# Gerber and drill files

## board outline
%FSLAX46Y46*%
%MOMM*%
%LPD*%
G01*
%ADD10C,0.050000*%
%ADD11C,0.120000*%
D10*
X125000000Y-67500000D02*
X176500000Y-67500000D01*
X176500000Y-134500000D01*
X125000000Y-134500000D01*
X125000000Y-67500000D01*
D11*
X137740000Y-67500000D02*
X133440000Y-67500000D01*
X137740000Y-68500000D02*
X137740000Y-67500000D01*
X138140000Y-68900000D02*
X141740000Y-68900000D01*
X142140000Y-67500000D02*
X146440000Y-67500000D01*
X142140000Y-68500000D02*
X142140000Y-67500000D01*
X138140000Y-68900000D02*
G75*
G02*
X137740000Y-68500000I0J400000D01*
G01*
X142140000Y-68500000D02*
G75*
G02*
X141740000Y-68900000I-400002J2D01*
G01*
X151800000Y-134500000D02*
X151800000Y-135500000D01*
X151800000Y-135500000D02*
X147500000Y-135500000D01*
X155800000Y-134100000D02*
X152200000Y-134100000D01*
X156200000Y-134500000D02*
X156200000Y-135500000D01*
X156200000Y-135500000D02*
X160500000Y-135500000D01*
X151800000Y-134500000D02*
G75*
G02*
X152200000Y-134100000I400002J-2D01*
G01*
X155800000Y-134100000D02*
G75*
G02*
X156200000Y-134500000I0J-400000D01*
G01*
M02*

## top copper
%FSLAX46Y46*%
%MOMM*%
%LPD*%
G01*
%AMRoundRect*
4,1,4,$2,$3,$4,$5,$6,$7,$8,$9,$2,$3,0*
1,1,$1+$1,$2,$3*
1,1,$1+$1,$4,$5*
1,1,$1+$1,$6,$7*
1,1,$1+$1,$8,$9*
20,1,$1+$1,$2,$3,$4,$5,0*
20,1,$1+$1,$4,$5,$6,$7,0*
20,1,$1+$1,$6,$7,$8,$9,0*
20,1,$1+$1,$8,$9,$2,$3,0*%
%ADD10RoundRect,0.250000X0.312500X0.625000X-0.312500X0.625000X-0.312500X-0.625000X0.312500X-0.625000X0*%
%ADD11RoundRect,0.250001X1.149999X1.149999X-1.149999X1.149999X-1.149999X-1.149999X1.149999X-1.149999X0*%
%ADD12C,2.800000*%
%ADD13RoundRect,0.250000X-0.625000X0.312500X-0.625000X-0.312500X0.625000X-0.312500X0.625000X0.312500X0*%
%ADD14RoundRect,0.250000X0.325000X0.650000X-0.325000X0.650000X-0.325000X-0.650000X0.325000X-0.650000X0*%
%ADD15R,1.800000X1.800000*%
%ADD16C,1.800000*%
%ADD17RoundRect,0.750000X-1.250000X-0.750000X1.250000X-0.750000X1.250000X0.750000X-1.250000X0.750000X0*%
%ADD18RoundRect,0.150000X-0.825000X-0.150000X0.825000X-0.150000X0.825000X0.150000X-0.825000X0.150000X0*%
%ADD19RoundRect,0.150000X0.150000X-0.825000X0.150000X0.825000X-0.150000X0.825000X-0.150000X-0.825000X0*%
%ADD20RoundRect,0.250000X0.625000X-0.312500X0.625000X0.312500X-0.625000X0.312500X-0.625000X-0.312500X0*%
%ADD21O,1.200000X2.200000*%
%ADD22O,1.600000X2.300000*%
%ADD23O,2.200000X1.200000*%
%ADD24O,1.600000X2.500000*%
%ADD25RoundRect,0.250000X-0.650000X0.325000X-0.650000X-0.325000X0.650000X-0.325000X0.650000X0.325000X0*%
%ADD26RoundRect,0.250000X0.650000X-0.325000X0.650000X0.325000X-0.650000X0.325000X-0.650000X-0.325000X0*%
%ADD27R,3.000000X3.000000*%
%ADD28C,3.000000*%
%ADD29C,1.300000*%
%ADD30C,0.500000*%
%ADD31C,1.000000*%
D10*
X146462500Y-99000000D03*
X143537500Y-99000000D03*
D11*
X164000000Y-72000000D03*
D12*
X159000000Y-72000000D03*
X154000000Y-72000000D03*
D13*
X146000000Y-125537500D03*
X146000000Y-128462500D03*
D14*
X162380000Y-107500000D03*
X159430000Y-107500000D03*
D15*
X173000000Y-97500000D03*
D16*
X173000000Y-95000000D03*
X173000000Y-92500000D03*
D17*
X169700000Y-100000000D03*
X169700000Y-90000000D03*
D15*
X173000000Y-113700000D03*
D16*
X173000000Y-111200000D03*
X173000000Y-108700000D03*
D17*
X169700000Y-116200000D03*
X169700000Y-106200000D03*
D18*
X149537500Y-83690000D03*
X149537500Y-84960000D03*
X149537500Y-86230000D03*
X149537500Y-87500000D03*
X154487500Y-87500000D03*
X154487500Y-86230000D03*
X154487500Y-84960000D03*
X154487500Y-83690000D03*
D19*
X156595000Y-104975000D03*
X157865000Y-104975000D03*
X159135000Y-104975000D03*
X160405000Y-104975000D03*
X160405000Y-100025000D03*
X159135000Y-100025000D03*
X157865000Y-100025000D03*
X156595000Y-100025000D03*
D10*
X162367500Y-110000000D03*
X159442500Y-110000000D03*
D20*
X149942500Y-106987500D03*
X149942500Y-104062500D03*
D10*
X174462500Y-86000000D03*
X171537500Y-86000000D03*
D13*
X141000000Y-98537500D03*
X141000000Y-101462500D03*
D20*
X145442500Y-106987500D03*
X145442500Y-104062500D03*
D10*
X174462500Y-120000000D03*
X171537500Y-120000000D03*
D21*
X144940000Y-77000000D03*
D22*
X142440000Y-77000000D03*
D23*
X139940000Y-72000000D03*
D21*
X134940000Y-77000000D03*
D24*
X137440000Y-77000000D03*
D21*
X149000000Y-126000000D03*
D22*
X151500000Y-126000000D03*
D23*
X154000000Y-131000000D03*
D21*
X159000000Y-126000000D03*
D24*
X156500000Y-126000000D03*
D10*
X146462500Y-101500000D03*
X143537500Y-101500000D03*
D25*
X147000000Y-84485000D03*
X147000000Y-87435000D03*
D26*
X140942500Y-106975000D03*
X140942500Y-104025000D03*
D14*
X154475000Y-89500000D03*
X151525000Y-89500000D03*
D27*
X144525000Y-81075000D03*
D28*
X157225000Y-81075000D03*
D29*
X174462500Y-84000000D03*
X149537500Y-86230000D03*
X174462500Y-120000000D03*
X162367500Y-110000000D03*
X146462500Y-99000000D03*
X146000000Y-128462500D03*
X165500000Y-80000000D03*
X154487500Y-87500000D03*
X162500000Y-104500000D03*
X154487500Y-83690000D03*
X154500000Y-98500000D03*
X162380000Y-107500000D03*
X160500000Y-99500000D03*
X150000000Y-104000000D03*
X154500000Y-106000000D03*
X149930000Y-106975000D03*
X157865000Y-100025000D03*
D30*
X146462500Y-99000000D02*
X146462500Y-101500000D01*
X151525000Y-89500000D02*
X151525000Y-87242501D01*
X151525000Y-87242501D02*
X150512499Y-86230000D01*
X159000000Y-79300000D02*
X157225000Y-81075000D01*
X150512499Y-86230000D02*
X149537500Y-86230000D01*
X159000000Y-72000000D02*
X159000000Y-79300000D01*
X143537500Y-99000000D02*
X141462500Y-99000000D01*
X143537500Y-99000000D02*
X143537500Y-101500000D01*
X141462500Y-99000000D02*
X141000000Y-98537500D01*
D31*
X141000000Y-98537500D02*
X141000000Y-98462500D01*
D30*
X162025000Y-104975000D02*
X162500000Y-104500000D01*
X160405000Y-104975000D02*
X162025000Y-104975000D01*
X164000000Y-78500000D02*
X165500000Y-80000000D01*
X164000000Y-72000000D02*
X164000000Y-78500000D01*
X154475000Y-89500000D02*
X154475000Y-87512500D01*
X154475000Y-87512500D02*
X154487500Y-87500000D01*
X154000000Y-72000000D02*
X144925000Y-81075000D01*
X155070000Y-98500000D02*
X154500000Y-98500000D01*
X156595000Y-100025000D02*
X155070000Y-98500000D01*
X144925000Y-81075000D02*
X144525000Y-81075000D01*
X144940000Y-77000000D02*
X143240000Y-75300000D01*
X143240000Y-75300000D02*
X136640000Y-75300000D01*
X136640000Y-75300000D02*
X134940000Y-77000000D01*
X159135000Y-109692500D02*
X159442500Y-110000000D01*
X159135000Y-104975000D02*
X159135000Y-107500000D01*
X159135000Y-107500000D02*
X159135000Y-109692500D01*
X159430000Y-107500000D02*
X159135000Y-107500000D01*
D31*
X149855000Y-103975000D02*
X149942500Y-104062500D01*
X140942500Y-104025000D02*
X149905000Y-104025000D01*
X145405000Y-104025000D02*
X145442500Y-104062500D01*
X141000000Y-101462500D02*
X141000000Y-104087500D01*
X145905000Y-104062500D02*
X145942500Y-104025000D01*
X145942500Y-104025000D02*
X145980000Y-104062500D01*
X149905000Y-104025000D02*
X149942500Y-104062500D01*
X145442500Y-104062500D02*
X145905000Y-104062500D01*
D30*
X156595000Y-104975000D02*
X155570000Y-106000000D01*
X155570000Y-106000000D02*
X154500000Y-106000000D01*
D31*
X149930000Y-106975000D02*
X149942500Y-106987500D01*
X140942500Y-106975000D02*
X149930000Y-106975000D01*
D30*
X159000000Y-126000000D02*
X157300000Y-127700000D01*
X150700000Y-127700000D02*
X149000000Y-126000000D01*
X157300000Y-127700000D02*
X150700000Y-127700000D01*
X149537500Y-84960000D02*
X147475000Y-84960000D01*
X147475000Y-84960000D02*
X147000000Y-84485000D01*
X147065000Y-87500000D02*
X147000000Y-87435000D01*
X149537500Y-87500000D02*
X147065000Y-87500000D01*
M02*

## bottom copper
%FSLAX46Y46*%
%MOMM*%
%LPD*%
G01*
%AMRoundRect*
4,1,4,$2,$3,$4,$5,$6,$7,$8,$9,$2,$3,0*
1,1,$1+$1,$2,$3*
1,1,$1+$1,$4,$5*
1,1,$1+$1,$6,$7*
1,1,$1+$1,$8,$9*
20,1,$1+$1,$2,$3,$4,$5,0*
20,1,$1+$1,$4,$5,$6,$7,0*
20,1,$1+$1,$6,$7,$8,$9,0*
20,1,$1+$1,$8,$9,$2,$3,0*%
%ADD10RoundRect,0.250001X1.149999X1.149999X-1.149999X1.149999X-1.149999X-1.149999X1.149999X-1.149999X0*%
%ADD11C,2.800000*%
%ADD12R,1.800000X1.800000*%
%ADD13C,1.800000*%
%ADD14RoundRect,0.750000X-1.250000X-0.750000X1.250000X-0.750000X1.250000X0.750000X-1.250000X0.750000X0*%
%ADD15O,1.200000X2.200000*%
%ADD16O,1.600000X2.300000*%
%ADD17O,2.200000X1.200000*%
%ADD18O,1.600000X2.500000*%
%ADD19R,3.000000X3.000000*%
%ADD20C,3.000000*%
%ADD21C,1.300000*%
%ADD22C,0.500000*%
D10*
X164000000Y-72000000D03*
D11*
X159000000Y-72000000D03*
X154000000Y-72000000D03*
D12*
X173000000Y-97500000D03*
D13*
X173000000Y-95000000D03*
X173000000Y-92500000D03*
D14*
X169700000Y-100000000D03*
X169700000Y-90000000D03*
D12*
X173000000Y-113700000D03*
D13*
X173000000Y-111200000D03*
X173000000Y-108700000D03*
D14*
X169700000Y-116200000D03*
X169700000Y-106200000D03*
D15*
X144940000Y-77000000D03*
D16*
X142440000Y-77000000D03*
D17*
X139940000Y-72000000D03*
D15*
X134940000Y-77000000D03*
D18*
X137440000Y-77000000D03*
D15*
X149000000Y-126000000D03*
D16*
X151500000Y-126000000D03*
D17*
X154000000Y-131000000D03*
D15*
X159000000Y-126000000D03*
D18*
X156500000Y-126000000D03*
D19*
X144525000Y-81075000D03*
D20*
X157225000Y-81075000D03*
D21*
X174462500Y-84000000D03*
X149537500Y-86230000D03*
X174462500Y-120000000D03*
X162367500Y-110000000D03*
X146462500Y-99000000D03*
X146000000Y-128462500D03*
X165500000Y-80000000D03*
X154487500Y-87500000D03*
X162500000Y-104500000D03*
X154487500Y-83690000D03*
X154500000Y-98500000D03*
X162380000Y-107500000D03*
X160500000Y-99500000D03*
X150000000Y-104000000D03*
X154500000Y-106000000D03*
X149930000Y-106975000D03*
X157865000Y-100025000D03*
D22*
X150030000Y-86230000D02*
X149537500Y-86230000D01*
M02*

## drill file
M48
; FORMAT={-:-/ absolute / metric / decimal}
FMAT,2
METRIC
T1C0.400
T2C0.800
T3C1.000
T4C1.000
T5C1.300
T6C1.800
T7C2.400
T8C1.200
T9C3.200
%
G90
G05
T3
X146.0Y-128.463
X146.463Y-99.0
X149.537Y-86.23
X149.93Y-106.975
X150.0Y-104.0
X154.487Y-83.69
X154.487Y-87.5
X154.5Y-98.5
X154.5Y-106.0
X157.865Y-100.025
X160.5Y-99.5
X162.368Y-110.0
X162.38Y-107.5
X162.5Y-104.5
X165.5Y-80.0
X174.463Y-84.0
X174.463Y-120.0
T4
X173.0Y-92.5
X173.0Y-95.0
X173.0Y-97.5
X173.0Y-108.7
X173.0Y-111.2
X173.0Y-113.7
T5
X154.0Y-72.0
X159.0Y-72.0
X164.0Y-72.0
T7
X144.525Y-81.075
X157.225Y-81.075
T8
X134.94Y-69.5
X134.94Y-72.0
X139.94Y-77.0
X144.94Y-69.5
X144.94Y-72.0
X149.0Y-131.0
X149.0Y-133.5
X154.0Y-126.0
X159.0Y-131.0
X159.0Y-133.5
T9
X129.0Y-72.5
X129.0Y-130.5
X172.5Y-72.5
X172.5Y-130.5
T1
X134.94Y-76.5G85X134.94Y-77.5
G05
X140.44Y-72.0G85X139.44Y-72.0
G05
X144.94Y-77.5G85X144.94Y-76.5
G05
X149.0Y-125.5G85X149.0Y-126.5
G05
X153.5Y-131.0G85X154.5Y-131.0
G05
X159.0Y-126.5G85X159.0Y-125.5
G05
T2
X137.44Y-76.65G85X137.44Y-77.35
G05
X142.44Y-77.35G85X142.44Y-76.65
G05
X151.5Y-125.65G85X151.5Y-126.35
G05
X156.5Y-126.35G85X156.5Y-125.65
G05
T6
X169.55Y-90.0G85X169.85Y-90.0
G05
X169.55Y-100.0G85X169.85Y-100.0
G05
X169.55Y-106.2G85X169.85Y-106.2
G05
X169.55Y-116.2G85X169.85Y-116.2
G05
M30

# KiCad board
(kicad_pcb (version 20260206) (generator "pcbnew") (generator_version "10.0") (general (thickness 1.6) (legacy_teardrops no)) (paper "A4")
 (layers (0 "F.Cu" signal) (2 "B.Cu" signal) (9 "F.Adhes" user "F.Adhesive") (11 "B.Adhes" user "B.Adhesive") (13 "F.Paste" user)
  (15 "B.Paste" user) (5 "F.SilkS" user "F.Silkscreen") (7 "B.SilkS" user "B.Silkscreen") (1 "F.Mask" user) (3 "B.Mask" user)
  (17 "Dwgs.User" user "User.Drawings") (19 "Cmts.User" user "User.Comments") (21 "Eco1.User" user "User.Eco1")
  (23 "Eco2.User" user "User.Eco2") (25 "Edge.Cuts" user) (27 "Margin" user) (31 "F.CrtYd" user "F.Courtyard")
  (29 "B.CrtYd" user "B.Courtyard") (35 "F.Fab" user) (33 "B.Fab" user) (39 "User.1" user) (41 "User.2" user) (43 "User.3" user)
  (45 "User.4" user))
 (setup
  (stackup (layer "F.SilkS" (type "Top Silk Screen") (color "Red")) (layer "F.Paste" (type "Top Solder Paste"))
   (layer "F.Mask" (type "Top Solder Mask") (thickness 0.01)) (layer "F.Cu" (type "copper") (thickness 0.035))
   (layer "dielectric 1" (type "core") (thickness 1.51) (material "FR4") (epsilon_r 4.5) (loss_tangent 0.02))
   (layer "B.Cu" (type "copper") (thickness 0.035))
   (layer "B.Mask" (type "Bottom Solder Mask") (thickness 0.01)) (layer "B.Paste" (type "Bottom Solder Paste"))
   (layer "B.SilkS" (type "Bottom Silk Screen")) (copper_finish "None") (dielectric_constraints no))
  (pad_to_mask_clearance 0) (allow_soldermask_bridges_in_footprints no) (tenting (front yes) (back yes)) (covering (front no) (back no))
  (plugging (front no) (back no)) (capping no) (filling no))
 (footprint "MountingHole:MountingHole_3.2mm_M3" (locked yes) (layer "F.Cu") (at 172.5 130.5)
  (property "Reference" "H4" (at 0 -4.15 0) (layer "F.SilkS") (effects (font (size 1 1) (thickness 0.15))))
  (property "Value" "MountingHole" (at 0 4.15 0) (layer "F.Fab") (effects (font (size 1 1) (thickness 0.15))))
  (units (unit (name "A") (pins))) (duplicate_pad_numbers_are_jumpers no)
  (pad "" np_thru_hole circle (at 0 0) (size 3.2 3.2) (drill 3.2) (layers "*.Cu" "*.Mask")))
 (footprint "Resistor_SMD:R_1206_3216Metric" (layer "F.Cu") (at 145 99 180)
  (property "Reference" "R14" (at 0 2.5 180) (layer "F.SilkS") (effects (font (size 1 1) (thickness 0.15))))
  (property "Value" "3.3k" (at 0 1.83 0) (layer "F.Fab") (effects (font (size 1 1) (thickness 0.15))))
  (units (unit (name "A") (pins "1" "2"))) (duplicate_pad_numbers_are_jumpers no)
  (pad "1" smd roundrect (at -1.4625 0 180) (size 1.125 1.75) (layers "F.Cu" "F.Mask" "F.Paste") (roundrect_rratio 0.222222) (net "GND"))
  (pad "2" smd roundrect (at 1.4625 0 180) (size 1.125 1.75) (layers "F.Cu" "F.Mask" "F.Paste") (roundrect_rratio 0.222222)
   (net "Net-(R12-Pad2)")))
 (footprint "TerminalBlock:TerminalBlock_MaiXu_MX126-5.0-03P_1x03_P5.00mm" (layer "F.Cu") (at 164 72 180)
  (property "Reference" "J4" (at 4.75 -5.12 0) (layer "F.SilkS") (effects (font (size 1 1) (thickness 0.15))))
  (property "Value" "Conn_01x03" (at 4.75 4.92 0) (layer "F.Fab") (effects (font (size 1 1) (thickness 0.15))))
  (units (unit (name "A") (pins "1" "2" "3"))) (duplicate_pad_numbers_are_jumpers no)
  (pad "1" thru_hole roundrect (at 0 0 180) (size 2.8 2.8) (drill 1.3) (layers "*.Cu" "*.Mask") (remove_unused_layers no)
   (roundrect_rratio 0.089286) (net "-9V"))
  (pad "2" thru_hole circle (at 5 0 180) (size 2.8 2.8) (drill 1.3) (layers "*.Cu" "*.Mask") (remove_unused_layers no) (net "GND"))
  (pad "3" thru_hole circle (at 10 0 180) (size 2.8 2.8) (drill 1.3) (layers "*.Cu" "*.Mask") (remove_unused_layers no) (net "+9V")))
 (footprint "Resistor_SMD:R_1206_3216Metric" (layer "F.Cu") (at 146 127 -90)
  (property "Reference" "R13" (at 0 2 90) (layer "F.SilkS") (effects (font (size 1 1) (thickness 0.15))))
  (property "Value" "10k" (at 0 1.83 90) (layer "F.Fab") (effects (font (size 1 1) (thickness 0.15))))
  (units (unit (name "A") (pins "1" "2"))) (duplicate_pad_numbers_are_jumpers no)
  (pad "1" smd roundrect (at -1.4625 0 270) (size 1.125 1.75) (layers "F.Cu" "F.Mask" "F.Paste") (roundrect_rratio 0.222222) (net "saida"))
  (pad "2" smd roundrect (at 1.4625 0 270) (size 1.125 1.75) (layers "F.Cu" "F.Mask" "F.Paste") (roundrect_rratio 0.222222) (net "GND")))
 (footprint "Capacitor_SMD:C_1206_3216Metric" (layer "F.Cu") (at 160.905 107.5 180)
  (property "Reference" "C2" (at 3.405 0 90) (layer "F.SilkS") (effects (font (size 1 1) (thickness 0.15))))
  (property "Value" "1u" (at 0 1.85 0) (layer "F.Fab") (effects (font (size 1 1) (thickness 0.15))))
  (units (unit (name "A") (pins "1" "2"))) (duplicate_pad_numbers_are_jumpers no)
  (pad "1" smd roundrect (at -1.475 0 180) (size 1.15 1.8) (layers "F.Cu" "F.Mask" "F.Paste") (roundrect_rratio 0.217391) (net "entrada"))
  (pad "2" smd roundrect (at 1.475 0 180) (size 1.15 1.8) (layers "F.Cu" "F.Mask" "F.Paste") (roundrect_rratio 0.217391) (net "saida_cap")))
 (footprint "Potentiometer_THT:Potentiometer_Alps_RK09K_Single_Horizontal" (layer "F.Cu") (at 173 97.5 180)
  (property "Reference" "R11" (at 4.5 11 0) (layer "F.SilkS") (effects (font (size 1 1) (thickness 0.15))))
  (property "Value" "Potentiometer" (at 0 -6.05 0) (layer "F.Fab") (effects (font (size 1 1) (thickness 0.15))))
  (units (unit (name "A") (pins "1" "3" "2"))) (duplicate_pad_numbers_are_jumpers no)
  (pad "1" thru_hole rect (at 0 0) (size 1.8 1.8) (drill 1) (layers "*.Cu" "*.Mask") (remove_unused_layers no) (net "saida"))
  (pad "2" thru_hole circle (at 0 2.5) (size 1.8 1.8) (drill 1) (layers "*.Cu" "*.Mask") (remove_unused_layers no) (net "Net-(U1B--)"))
  (pad "3" thru_hole circle (at 0 5) (size 1.8 1.8) (drill 1) (layers "*.Cu" "*.Mask") (remove_unused_layers no)
   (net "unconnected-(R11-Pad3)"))
  (pad "MP" thru_hole roundrect (at 3.3 -2.5) (size 4 3) (drill oval 2.1 1.8) (layers "*.Cu" "*.Mask") (remove_unused_layers no)
   (roundrect_rratio 0.25))
  (pad "MP" thru_hole roundrect (at 3.3 7.5) (size 4 3) (drill oval 2.1 1.8) (layers "*.Cu" "*.Mask") (remove_unused_layers no)
   (roundrect_rratio 0.25))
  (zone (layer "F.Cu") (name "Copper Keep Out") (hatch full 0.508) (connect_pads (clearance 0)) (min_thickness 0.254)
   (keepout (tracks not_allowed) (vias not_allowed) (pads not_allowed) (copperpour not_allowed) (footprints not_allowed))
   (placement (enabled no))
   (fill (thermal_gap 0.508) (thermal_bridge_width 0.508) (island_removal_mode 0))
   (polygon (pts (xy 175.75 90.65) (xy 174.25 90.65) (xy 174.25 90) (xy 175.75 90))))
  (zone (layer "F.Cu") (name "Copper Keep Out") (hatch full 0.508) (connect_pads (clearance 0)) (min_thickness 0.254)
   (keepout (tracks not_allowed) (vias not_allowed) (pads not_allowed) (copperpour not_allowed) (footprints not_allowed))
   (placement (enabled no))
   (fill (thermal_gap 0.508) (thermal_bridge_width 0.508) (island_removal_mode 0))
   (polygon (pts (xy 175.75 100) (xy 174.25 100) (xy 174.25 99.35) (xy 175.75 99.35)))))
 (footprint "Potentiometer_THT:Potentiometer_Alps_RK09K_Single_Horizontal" (layer "F.Cu") (at 173 113.7 180)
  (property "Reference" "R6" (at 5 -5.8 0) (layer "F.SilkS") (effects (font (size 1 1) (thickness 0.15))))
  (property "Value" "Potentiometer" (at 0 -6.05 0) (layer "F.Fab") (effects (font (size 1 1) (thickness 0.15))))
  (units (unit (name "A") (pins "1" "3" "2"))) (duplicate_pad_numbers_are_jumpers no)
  (pad "1" thru_hole rect (at 0 0) (size 1.8 1.8) (drill 1) (layers "*.Cu" "*.Mask") (remove_unused_layers no) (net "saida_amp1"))
  (pad "2" thru_hole circle (at 0 2.5) (size 1.8 1.8) (drill 1) (layers "*.Cu" "*.Mask") (remove_unused_layers no) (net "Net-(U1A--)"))
  (pad "3" thru_hole circle (at 0 5) (size 1.8 1.8) (drill 1) (layers "*.Cu" "*.Mask") (remove_unused_layers no)
   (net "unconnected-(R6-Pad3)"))
  (pad "MP" thru_hole roundrect (at 3.3 -2.5) (size 4 3) (drill oval 2.1 1.8) (layers "*.Cu" "*.Mask") (remove_unused_layers no)
   (roundrect_rratio 0.25))
  (pad "MP" thru_hole roundrect (at 3.3 7.5) (size 4 3) (drill oval 2.1 1.8) (layers "*.Cu" "*.Mask") (remove_unused_layers no)
   (roundrect_rratio 0.25))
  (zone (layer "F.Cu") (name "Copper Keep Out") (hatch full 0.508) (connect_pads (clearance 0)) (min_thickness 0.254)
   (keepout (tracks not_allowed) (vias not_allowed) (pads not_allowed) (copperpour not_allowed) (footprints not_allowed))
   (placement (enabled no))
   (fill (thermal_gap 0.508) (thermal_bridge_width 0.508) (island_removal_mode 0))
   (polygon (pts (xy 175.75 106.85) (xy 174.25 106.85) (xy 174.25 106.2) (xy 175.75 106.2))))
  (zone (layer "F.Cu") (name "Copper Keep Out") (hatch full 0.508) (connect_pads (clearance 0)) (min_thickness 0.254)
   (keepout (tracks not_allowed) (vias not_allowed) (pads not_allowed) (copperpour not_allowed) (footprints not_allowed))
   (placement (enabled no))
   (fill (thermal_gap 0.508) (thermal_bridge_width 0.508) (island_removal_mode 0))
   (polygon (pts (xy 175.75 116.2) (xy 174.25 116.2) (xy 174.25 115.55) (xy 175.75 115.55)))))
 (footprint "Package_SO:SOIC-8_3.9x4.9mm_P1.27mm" (layer "F.Cu") (at 152.0125 85.595)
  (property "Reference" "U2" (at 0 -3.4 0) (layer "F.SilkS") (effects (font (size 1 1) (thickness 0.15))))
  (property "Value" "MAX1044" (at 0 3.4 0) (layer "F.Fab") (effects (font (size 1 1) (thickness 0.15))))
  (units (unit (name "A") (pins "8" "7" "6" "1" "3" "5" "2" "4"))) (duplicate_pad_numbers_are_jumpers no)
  (pad "1" smd roundrect (at -2.475 -1.905) (size 1.95 0.6) (layers "F.Cu" "F.Mask" "F.Paste") (roundrect_rratio 0.25)
   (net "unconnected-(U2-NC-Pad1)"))
  (pad "2" smd roundrect (at -2.475 -0.635) (size 1.95 0.6) (layers "F.Cu" "F.Mask" "F.Paste") (roundrect_rratio 0.25) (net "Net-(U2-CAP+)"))
  (pad "3" smd roundrect (at -2.475 0.635) (size 1.95 0.6) (layers "F.Cu" "F.Mask" "F.Paste") (roundrect_rratio 0.25) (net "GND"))
  (pad "4" smd roundrect (at -2.475 1.905) (size 1.95 0.6) (layers "F.Cu" "F.Mask" "F.Paste") (roundrect_rratio 0.25) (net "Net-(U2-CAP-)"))
  (pad "5" smd roundrect (at 2.475 1.905) (size 1.95 0.6) (layers "F.Cu" "F.Mask" "F.Paste") (roundrect_rratio 0.25) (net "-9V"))
  (pad "6" smd roundrect (at 2.475 0.635) (size 1.95 0.6) (layers "F.Cu" "F.Mask" "F.Paste") (roundrect_rratio 0.25)
   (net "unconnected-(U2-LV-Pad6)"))
  (pad "7" smd roundrect (at 2.475 -0.635) (size 1.95 0.6) (layers "F.Cu" "F.Mask" "F.Paste") (roundrect_rratio 0.25)
   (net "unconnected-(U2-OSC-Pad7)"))
  (pad "8" smd roundrect (at 2.475 -1.905) (size 1.95 0.6) (layers "F.Cu" "F.Mask" "F.Paste") (roundrect_rratio 0.25) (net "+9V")))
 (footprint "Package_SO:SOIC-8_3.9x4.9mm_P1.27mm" (layer "F.Cu") (at 158.5 102.5 90)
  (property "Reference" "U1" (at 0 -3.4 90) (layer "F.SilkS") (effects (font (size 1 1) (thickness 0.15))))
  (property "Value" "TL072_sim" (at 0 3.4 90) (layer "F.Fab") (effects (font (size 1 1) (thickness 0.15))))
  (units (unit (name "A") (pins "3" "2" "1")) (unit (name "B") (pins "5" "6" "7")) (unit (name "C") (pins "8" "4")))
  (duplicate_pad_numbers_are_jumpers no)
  (pad "1" smd roundrect (at -2.475 -1.905 90) (size 1.95 0.6) (layers "F.Cu" "F.Mask" "F.Paste") (roundrect_rratio 0.25) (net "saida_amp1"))
  (pad "2" smd roundrect (at -2.475 -0.635 90) (size 1.95 0.6) (layers "F.Cu" "F.Mask" "F.Paste") (roundrect_rratio 0.25)
   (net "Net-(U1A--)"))
  (pad "3" smd roundrect (at -2.475 0.635 90) (size 1.95 0.6) (layers "F.Cu" "F.Mask" "F.Paste") (roundrect_rratio 0.25) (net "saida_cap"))
  (pad "4" smd roundrect (at -2.475 1.905 90) (size 1.95 0.6) (layers "F.Cu" "F.Mask" "F.Paste") (roundrect_rratio 0.25) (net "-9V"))
  (pad "5" smd roundrect (at 2.475 1.905 90) (size 1.95 0.6) (layers "F.Cu" "F.Mask" "F.Paste") (roundrect_rratio 0.25) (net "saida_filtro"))
  (pad "6" smd roundrect (at 2.475 0.635 90) (size 1.95 0.6) (layers "F.Cu" "F.Mask" "F.Paste") (roundrect_rratio 0.25) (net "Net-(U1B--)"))
  (pad "7" smd roundrect (at 2.475 -0.635 90) (size 1.95 0.6) (layers "F.Cu" "F.Mask" "F.Paste") (roundrect_rratio 0.25) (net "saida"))
  (pad "8" smd roundrect (at 2.475 -1.905 90) (size 1.95 0.6) (layers "F.Cu" "F.Mask" "F.Paste") (roundrect_rratio 0.25) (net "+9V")))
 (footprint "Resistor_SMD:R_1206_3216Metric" (layer "F.Cu") (at 160.905 110 180)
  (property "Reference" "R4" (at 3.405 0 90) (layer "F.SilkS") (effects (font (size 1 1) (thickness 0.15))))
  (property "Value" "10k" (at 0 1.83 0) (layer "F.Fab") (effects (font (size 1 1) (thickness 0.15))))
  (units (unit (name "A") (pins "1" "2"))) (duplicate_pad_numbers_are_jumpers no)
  (pad "1" smd roundrect (at -1.4625 0 180) (size 1.125 1.75) (layers "F.Cu" "F.Mask" "F.Paste") (roundrect_rratio 0.222222) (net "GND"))
  (pad "2" smd roundrect (at 1.4625 0 180) (size 1.125 1.75) (layers "F.Cu" "F.Mask" "F.Paste") (roundrect_rratio 0.222222)
   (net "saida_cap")))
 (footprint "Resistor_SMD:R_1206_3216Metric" (layer "F.Cu") (at 149.9425 105.525 90)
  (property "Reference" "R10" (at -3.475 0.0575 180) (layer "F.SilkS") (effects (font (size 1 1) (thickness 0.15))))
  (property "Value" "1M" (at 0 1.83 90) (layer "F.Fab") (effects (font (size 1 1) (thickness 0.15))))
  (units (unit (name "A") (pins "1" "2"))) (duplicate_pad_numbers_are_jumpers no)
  (pad "1" smd roundrect (at -1.4625 0 90) (size 1.125 1.75) (layers "F.Cu" "F.Mask" "F.Paste") (roundrect_rratio 0.222222)
   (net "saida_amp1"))
  (pad "2" smd roundrect (at 1.4625 0 90) (size 1.125 1.75) (layers "F.Cu" "F.Mask" "F.Paste") (roundrect_rratio 0.222222)
   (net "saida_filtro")))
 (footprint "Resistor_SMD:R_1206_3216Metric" (layer "F.Cu") (at 173 86 180)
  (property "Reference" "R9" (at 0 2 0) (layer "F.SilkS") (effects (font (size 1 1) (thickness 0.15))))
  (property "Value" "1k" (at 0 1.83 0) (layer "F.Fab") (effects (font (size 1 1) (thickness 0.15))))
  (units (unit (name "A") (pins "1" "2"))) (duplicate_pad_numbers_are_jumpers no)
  (pad "1" smd roundrect (at -1.4625 0 180) (size 1.125 1.75) (layers "F.Cu" "F.Mask" "F.Paste") (roundrect_rratio 0.222222) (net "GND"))
  (pad "2" smd roundrect (at 1.4625 0 180) (size 1.125 1.75) (layers "F.Cu" "F.Mask" "F.Paste") (roundrect_rratio 0.222222)
   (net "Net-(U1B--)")))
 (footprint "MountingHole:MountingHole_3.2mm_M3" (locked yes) (layer "F.Cu") (at 172.5 72.5)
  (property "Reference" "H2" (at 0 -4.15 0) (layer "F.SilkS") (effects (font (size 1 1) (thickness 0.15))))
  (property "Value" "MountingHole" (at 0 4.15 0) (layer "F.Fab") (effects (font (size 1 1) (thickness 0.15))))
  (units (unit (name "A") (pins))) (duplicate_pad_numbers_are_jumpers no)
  (pad "" np_thru_hole circle (at 0 0) (size 3.2 3.2) (drill 3.2) (layers "*.Cu" "*.Mask")))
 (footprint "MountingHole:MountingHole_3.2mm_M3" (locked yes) (layer "F.Cu") (at 129 72.5)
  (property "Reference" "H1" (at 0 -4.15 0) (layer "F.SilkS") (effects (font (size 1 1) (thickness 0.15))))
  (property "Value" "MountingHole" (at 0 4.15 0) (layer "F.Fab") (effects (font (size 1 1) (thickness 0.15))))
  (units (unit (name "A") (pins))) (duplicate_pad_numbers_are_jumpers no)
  (pad "" np_thru_hole circle (at 0 0) (size 3.2 3.2) (drill 3.2) (layers "*.Cu" "*.Mask")))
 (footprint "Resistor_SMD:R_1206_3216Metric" (layer "F.Cu") (at 141 100 -90)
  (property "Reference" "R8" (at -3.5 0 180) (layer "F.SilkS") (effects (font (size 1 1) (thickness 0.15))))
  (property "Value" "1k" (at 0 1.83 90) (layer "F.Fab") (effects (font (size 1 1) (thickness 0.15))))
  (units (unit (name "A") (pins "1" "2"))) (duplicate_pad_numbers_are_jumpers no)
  (pad "1" smd roundrect (at -1.4625 0 270) (size 1.125 1.75) (layers "F.Cu" "F.Mask" "F.Paste") (roundrect_rratio 0.222222)
   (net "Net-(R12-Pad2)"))
  (pad "2" smd roundrect (at 1.4625 0 270) (size 1.125 1.75) (layers "F.Cu" "F.Mask" "F.Paste") (roundrect_rratio 0.222222)
   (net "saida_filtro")))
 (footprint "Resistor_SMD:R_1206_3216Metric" (layer "F.Cu") (at 145.4425 105.525 90)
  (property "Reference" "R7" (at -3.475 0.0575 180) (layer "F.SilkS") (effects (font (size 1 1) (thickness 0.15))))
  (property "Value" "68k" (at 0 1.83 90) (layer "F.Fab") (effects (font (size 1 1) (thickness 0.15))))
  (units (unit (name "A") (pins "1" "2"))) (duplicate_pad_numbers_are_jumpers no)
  (pad "1" smd roundrect (at -1.4625 0 90) (size 1.125 1.75) (layers "F.Cu" "F.Mask" "F.Paste") (roundrect_rratio 0.222222)
   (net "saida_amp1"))
  (pad "2" smd roundrect (at 1.4625 0 90) (size 1.125 1.75) (layers "F.Cu" "F.Mask" "F.Paste") (roundrect_rratio 0.222222)
   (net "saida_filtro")))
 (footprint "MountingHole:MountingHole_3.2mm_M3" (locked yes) (layer "F.Cu") (at 129 130.5)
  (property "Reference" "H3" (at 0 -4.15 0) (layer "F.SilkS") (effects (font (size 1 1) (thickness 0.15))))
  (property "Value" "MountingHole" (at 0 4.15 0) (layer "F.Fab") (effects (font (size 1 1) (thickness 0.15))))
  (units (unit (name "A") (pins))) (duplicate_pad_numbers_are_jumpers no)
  (pad "" np_thru_hole circle (at 0 0) (size 3.2 3.2) (drill 3.2) (layers "*.Cu" "*.Mask")))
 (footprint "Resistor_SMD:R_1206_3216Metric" (layer "F.Cu") (at 173 120 180)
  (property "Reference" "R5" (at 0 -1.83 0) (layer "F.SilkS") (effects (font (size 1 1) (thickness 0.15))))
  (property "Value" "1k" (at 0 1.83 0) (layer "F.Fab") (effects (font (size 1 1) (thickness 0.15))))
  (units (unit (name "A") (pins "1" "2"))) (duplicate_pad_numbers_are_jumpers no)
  (pad "1" smd roundrect (at -1.4625 0 180) (size 1.125 1.75) (layers "F.Cu" "F.Mask" "F.Paste") (roundrect_rratio 0.222222) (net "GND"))
  (pad "2" smd roundrect (at 1.4625 0 180) (size 1.125 1.75) (layers "F.Cu" "F.Mask" "F.Paste") (roundrect_rratio 0.222222)
   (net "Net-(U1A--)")))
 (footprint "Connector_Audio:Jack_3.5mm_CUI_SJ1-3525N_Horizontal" (layer "F.Cu") (at 139.94 72 180)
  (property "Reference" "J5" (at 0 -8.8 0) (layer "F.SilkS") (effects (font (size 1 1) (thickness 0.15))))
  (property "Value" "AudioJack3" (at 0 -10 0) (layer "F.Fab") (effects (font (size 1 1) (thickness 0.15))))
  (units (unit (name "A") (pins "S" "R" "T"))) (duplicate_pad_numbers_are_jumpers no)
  (fp_line (start 2.2 4.5) (end 6.5 4.5) (stroke (width 0.12) (type solid)) (layer "Edge.Cuts"))
  (fp_line (start 2.2 3.5) (end 2.2 4.5) (stroke (width 0.12) (type solid)) (layer "Edge.Cuts"))
  (fp_line (start 1.8 3.1) (end -1.8 3.1) (stroke (width 0.12) (type solid)) (layer "Edge.Cuts"))
  (fp_line (start -2.2 4.5) (end -6.5 4.5) (stroke (width 0.12) (type solid)) (layer "Edge.Cuts"))
  (fp_line (start -2.2 3.5) (end -2.2 4.5) (stroke (width 0.12) (type solid)) (layer "Edge.Cuts"))
  (fp_arc (start 1.8 3.1) (mid 2.082843 3.217157) (end 2.2 3.5) (stroke (width 0.12) (type solid)) (layer "Edge.Cuts"))
  (fp_arc (start -2.2 3.5) (mid -2.082842 3.217158) (end -1.8 3.1) (stroke (width 0.12) (type solid)) (layer "Edge.Cuts"))
  (pad "" np_thru_hole circle (at -5 0 180) (size 1.2 1.2) (drill 1.2) (layers "*.Cu" "*.Mask"))
  (pad "" np_thru_hole circle (at -5 2.5 180) (size 1.2 1.2) (drill 1.2) (layers "*.Cu" "*.Mask"))
  (pad "" np_thru_hole circle (at 0 -5 180) (size 1.2 1.2) (drill 1.2) (layers "*.Cu" "*.Mask"))
  (pad "" np_thru_hole circle (at 5 0 180) (size 1.2 1.2) (drill 1.2) (layers "*.Cu" "*.Mask"))
  (pad "" np_thru_hole circle (at 5 2.5 180) (size 1.2 1.2) (drill 1.2) (layers "*.Cu" "*.Mask"))
  (pad "R" thru_hole oval (at -5 -5 180) (size 1.2 2.2) (drill oval 0.4 1.4) (layers "*.Cu" "*.Mask") (remove_unused_layers no)
   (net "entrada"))
  (pad "RN" thru_hole oval (at -2.5 -5 180) (size 1.6 2.3) (drill oval 0.8 1.5) (layers "*.Cu" "*.Mask") (remove_unused_layers no))
  (pad "S" thru_hole oval (at 0 0 180) (size 2.2 1.2) (drill oval 1.4 0.4) (layers "*.Cu" "*.Mask") (remove_unused_layers no) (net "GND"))
  (pad "T" thru_hole oval (at 5 -5) (size 1.2 2.2) (drill oval 0.4 1.4) (layers "*.Cu" "*.Mask") (remove_unused_layers no) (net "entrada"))
  (pad "TN" thru_hole oval (at 2.5 -5) (size 1.6 2.5) (drill oval 0.8 1.5) (layers "*.Cu" "*.Mask") (remove_unused_layers no)))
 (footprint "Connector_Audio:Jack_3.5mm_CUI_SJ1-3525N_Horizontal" (layer "F.Cu") (at 154 131)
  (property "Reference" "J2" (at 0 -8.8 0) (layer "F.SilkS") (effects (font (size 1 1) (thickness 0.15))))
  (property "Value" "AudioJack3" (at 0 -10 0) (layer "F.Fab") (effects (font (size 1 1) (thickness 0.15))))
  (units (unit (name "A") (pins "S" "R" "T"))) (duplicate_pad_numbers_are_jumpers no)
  (fp_line (start -2.2 3.5) (end -2.2 4.5) (stroke (width 0.12) (type solid)) (layer "Edge.Cuts"))
  (fp_line (start -2.2 4.5) (end -6.5 4.5) (stroke (width 0.12) (type solid)) (layer "Edge.Cuts"))
  (fp_line (start 1.8 3.1) (end -1.8 3.1) (stroke (width 0.12) (type solid)) (layer "Edge.Cuts"))
  (fp_line (start 2.2 3.5) (end 2.2 4.5) (stroke (width 0.12) (type solid)) (layer "Edge.Cuts"))
  (fp_line (start 2.2 4.5) (end 6.5 4.5) (stroke (width 0.12) (type solid)) (layer "Edge.Cuts"))
  (fp_arc (start -2.2 3.5) (mid -2.082842 3.217158) (end -1.8 3.1) (stroke (width 0.12) (type solid)) (layer "Edge.Cuts"))
  (fp_arc (start 1.8 3.1) (mid 2.082843 3.217157) (end 2.2 3.5) (stroke (width 0.12) (type solid)) (layer "Edge.Cuts"))
  (pad "" np_thru_hole circle (at -5 0) (size 1.2 1.2) (drill 1.2) (layers "*.Cu" "*.Mask"))
  (pad "" np_thru_hole circle (at -5 2.5) (size 1.2 1.2) (drill 1.2) (layers "*.Cu" "*.Mask"))
  (pad "" np_thru_hole circle (at 0 -5) (size 1.2 1.2) (drill 1.2) (layers "*.Cu" "*.Mask"))
  (pad "" np_thru_hole circle (at 5 0) (size 1.2 1.2) (drill 1.2) (layers "*.Cu" "*.Mask"))
  (pad "" np_thru_hole circle (at 5 2.5) (size 1.2 1.2) (drill 1.2) (layers "*.Cu" "*.Mask"))
  (pad "R" thru_hole oval (at -5 -5) (size 1.2 2.2) (drill oval 0.4 1.4) (layers "*.Cu" "*.Mask") (remove_unused_layers no) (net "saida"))
  (pad "RN" thru_hole oval (at -2.5 -5) (size 1.6 2.3) (drill oval 0.8 1.5) (layers "*.Cu" "*.Mask") (remove_unused_layers no))
  (pad "S" thru_hole oval (at 0 0) (size 2.2 1.2) (drill oval 1.4 0.4) (layers "*.Cu" "*.Mask") (remove_unused_layers no) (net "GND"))
  (pad "T" thru_hole oval (at 5 -5 180) (size 1.2 2.2) (drill oval 0.4 1.4) (layers "*.Cu" "*.Mask") (remove_unused_layers no) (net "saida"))
  (pad "TN" thru_hole oval (at 2.5 -5 180) (size 1.6 2.5) (drill oval 0.8 1.5) (layers "*.Cu" "*.Mask") (remove_unused_layers no)))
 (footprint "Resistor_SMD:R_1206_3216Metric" (layer "F.Cu") (at 145 101.5 180)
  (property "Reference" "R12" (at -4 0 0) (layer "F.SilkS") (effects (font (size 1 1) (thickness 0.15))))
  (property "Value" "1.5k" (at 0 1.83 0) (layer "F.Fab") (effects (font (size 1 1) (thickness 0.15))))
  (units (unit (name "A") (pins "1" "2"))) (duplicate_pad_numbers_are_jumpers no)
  (pad "1" smd roundrect (at -1.4625 0 180) (size 1.125 1.75) (layers "F.Cu" "F.Mask" "F.Paste") (roundrect_rratio 0.222222) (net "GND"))
  (pad "2" smd roundrect (at 1.4625 0 180) (size 1.125 1.75) (layers "F.Cu" "F.Mask" "F.Paste") (roundrect_rratio 0.222222)
   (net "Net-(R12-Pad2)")))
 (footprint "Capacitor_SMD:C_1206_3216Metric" (layer "F.Cu") (at 147 85.96 -90)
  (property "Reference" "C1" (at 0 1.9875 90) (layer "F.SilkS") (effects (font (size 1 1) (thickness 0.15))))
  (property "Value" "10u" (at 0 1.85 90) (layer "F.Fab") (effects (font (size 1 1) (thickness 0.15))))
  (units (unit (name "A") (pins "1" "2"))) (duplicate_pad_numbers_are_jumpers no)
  (pad "1" smd roundrect (at -1.475 0 270) (size 1.15 1.8) (layers "F.Cu" "F.Mask" "F.Paste") (roundrect_rratio 0.217391)
   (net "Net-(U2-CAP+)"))
  (pad "2" smd roundrect (at 1.475 0 270) (size 1.15 1.8) (layers "F.Cu" "F.Mask" "F.Paste") (roundrect_rratio 0.217391)
   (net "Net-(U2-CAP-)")))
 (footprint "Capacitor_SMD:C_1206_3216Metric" (layer "F.Cu") (at 140.9425 105.5 90)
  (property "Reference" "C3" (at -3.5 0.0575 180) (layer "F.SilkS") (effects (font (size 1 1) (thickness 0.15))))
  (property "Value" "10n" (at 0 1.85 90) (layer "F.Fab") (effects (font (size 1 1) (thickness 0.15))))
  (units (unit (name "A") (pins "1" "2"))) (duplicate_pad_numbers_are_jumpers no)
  (pad "1" smd roundrect (at -1.475 0 90) (size 1.15 1.8) (layers "F.Cu" "F.Mask" "F.Paste") (roundrect_rratio 0.217391) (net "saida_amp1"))
  (pad "2" smd roundrect (at 1.475 0 90) (size 1.15 1.8) (layers "F.Cu" "F.Mask" "F.Paste") (roundrect_rratio 0.217391) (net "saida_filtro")))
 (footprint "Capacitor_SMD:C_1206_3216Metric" (layer "F.Cu") (at 153 89.5 180)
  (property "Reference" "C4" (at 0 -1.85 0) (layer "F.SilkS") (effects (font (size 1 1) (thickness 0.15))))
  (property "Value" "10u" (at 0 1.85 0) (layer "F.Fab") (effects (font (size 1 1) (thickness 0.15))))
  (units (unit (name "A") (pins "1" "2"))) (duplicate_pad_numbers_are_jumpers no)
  (pad "1" smd roundrect (at -1.475 0 180) (size 1.15 1.8) (layers "F.Cu" "F.Mask" "F.Paste") (roundrect_rratio 0.217391) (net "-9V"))
  (pad "2" smd roundrect (at 1.475 0 180) (size 1.15 1.8) (layers "F.Cu" "F.Mask" "F.Paste") (roundrect_rratio 0.217391) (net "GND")))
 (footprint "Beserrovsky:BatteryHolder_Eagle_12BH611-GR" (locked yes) (layer "B.Cu") (at 144.525 81.075 90)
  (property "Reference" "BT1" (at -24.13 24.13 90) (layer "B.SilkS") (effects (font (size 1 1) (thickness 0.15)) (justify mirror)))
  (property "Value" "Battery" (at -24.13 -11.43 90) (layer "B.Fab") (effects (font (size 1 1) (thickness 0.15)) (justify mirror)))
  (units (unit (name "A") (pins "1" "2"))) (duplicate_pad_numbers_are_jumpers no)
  (pad "1" thru_hole rect (at 0 0 90) (size 3 3) (drill 2.4) (layers "*.Cu" "*.Mask") (remove_unused_layers no) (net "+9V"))
  (pad "2" thru_hole circle (at 0 12.7 90) (size 3 3) (drill 2.4) (layers "*.Cu" "*.Mask") (remove_unused_layers no) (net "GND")))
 (gr_rect (start 125 67.5) (end 176.5 134.5) (stroke (width 0.05) (type default)) (fill no) (locked yes) (layer "Edge.Cuts"))
 (segment (start 146.4625 99) (end 146.4625 101.5) (width 0.5) (layer "F.Cu") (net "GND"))
 (segment (start 151.525 89.5) (end 151.525 87.242501) (width 0.5) (layer "F.Cu") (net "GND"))
 (segment (start 151.525 87.242501) (end 150.512499 86.23) (width 0.5) (layer "F.Cu") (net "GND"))
 (segment (start 159 79.3) (end 157.225 81.075) (width 0.5) (layer "F.Cu") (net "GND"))
 (segment (start 150.512499 86.23) (end 149.5375 86.23) (width 0.5) (layer "F.Cu") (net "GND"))
 (segment (start 159 72) (end 159 79.3) (width 0.5) (layer "F.Cu") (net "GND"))
 (via (at 174.4625 84) (size 1.3) (drill 1) (layers "F.Cu" "B.Cu") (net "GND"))
 (via (at 149.5375 86.23) (size 1.3) (drill 1) (layers "F.Cu" "B.Cu") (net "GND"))
 (via (at 174.4625 120) (size 1.3) (drill 1) (layers "F.Cu" "B.Cu") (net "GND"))
 (via (at 162.3675 110) (size 1.3) (drill 1) (layers "F.Cu" "B.Cu") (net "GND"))
 (via (at 146.4625 99) (size 1.3) (drill 1) (layers "F.Cu" "B.Cu") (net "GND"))
 (via (at 146 128.4625) (size 1.3) (drill 1) (layers "F.Cu" "B.Cu") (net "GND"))
 (segment (start 150.03 86.23) (end 149.5375 86.23) (width 0.5) (layer "B.Cu") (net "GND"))
 (segment (start 143.5375 99) (end 141.4625 99) (width 0.5) (layer "F.Cu") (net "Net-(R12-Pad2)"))
 (segment (start 143.5375 99) (end 143.5375 101.5) (width 0.5) (layer "F.Cu") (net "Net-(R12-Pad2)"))
 (segment (start 141.4625 99) (end 141 98.5375) (width 0.5) (layer "F.Cu") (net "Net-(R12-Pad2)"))
 (segment (start 141 98.5375) (end 141 98.4625) (width 1) (layer "F.Cu") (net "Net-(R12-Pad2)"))
 (segment (start 162.025 104.975) (end 162.5 104.5) (width 0.5) (layer "F.Cu") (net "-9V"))
 (segment (start 160.405 104.975) (end 162.025 104.975) (width 0.5) (layer "F.Cu") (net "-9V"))
 (segment (start 164 78.5) (end 165.5 80) (width 0.5) (layer "F.Cu") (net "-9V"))
 (segment (start 164 72) (end 164 78.5) (width 0.5) (layer "F.Cu") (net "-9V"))
 (segment (start 154.475 89.5) (end 154.475 87.5125) (width 0.5) (layer "F.Cu") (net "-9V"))
 (segment (start 154.475 87.5125) (end 154.4875 87.5) (width 0.5) (layer "F.Cu") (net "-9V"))
 (via (at 165.5 80) (size 1.3) (drill 1) (layers "F.Cu" "B.Cu") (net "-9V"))
 (via (at 154.4875 87.5) (size 1.3) (drill 1) (layers "F.Cu" "B.Cu") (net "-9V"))
 (via (at 162.5 104.5) (size 1.3) (drill 1) (layers "F.Cu" "B.Cu") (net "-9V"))
 (segment (start 154 72) (end 144.925 81.075) (width 0.5) (layer "F.Cu") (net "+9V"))
 (segment (start 155.07 98.5) (end 154.5 98.5) (width 0.5) (layer "F.Cu") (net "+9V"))
 (segment (start 156.595 100.025) (end 155.07 98.5) (width 0.5) (layer "F.Cu") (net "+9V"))
 (segment (start 144.925 81.075) (end 144.525 81.075) (width 0.5) (layer "F.Cu") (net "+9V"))
 (via (at 154.4875 83.69) (size 1.3) (drill 1) (layers "F.Cu" "B.Cu") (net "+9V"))
 (via (at 154.5 98.5) (size 1.3) (drill 1) (layers "F.Cu" "B.Cu") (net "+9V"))
 (segment (start 144.94 77) (end 143.24 75.3) (width 0.5) (layer "F.Cu") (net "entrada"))
 (segment (start 143.24 75.3) (end 136.64 75.3) (width 0.5) (layer "F.Cu") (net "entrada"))
 (segment (start 136.64 75.3) (end 134.94 77) (width 0.5) (layer "F.Cu") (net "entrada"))
 (via (at 162.38 107.5) (size 1.3) (drill 1) (layers "F.Cu" "B.Cu") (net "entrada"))
 (segment (start 159.135 109.6925) (end 159.4425 110) (width 0.5) (layer "F.Cu") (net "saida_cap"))
 (segment (start 159.135 104.975) (end 159.135 107.5) (width 0.5) (layer "F.Cu") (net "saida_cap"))
 (segment (start 159.135 107.5) (end 159.135 109.6925) (width 0.5) (layer "F.Cu") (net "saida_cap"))
 (segment (start 159.43 107.5) (end 159.135 107.5) (width 0.5) (layer "F.Cu") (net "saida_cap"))
 (segment (start 149.855 103.975) (end 149.9425 104.0625) (width 1) (layer "F.Cu") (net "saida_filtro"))
 (segment (start 140.9425 104.025) (end 149.905 104.025) (width 1) (layer "F.Cu") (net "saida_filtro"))
 (segment (start 145.405 104.025) (end 145.4425 104.0625) (width 1) (layer "F.Cu") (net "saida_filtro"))
 (segment (start 141 101.4625) (end 141 104.0875) (width 1) (layer "F.Cu") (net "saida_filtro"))
 (segment (start 145.905 104.0625) (end 145.9425 104.025) (width 1) (layer "F.Cu") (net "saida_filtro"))
 (segment (start 145.9425 104.025) (end 145.98 104.0625) (width 1) (layer "F.Cu") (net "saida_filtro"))
 (segment (start 149.905 104.025) (end 149.9425 104.0625) (width 1) (layer "F.Cu") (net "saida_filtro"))
 (segment (start 145.4425 104.0625) (end 145.905 104.0625) (width 1) (layer "F.Cu") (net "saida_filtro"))
 (via (at 160.5 99.5) (size 1.3) (drill 1) (layers "F.Cu" "B.Cu") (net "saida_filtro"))
 (via (at 150 104) (size 1.3) (drill 1) (layers "F.Cu" "B.Cu") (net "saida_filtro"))
 (segment (start 156.595 104.975) (end 155.57 106) (width 0.5) (layer "F.Cu") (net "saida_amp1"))
 (segment (start 155.57 106) (end 154.5 106) (width 0.5) (layer "F.Cu") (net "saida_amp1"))
 (segment (start 149.93 106.975) (end 149.9425 106.9875) (width 1) (layer "F.Cu") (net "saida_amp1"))
 (segment (start 140.9425 106.975) (end 149.93 106.975) (width 1) (layer "F.Cu") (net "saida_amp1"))
 (via (at 154.5 106) (size 1.3) (drill 1) (layers "F.Cu" "B.Cu") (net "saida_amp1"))
 (via (at 149.93 106.975) (size 1.3) (drill 1) (layers "F.Cu" "B.Cu") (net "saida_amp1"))
 (segment (start 159 126) (end 157.3 127.7) (width 0.5) (layer "F.Cu") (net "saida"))
 (segment (start 150.7 127.7) (end 149 126) (width 0.5) (layer "F.Cu") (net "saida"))
 (segment (start 157.3 127.7) (end 150.7 127.7) (width 0.5) (layer "F.Cu") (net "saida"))
 (via (at 157.865 100.025) (size 1.3) (drill 1) (layers "F.Cu" "B.Cu") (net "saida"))
 (segment (start 149.5375 84.96) (end 147.475 84.96) (width 0.5) (layer "F.Cu") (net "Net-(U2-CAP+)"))
 (segment (start 147.475 84.96) (end 147 84.485) (width 0.5) (layer "F.Cu") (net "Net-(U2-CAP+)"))
 (segment (start 147.065 87.5) (end 147 87.435) (width 0.5) (layer "F.Cu") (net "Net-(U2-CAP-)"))
 (segment (start 149.5375 87.5) (end 147.065 87.5) (width 0.5) (layer "F.Cu") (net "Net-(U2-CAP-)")))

